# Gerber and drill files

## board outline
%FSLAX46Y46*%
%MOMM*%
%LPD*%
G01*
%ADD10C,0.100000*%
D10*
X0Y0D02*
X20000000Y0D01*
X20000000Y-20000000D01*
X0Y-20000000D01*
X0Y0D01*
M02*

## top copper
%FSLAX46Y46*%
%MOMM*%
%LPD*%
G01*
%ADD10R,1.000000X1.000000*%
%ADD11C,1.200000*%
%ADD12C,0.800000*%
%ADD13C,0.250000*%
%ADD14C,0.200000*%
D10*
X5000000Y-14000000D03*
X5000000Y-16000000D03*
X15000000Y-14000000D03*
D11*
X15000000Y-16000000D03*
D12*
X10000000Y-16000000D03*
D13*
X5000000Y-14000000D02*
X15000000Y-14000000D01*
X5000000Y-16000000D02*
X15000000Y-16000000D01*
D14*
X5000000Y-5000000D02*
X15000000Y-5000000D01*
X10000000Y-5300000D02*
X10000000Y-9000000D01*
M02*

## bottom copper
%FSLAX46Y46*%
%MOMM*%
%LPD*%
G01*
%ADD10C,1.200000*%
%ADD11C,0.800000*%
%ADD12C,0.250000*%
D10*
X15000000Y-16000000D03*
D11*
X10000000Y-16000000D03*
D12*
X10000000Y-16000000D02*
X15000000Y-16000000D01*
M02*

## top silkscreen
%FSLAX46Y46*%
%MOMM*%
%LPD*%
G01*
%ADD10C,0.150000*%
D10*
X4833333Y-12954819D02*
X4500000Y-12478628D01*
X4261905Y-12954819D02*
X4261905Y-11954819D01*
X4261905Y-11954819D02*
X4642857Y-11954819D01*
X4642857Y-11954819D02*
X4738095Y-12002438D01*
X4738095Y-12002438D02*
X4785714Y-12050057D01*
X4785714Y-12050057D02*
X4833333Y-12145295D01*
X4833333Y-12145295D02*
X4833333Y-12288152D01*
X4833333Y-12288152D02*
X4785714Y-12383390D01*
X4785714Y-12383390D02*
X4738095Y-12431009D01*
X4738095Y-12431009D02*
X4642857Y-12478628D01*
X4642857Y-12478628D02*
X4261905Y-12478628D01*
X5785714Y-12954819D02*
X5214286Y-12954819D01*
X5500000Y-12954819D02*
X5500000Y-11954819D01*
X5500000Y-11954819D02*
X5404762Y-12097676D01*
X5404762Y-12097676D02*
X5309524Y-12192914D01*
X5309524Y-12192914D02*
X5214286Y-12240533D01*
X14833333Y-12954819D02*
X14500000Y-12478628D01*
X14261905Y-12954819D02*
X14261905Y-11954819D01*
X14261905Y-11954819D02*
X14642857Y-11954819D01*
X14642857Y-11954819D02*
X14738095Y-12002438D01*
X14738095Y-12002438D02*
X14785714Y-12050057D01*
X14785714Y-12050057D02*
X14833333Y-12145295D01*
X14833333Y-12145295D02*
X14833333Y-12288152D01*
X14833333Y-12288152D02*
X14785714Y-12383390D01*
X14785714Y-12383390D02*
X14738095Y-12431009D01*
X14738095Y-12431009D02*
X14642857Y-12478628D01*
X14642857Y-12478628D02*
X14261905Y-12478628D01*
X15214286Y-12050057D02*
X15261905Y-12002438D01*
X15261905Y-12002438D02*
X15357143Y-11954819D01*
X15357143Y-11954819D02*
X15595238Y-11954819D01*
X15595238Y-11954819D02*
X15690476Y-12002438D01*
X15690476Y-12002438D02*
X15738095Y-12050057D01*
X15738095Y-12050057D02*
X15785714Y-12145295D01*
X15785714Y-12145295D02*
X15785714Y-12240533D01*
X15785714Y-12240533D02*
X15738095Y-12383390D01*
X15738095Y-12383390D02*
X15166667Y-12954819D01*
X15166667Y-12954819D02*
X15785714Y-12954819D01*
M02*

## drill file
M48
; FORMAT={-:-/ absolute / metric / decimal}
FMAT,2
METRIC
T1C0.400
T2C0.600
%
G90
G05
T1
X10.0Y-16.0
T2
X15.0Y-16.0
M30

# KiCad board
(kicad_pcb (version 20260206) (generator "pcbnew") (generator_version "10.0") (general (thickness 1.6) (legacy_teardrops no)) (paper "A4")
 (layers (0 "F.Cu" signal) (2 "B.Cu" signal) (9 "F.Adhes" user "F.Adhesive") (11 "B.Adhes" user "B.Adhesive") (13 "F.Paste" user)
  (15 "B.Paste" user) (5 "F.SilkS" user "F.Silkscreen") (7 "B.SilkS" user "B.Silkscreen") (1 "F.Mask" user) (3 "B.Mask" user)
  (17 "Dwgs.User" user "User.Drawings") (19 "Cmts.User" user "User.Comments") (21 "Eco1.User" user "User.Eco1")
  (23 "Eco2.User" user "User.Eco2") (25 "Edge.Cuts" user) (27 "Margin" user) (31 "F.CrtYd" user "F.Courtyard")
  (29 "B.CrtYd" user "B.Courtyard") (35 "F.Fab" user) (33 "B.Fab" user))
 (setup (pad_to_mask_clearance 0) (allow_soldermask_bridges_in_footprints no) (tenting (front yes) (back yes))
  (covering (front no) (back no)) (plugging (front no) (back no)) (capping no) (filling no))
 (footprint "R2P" (layer "F.Cu") (at 5 15)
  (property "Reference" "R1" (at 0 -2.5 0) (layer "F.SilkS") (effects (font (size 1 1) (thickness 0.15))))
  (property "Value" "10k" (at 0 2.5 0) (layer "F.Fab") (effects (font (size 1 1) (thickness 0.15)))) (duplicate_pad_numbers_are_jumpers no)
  (pad "1" smd rect (at 0 -1) (size 1 1) (layers "F.Cu" "F.Mask" "F.Paste") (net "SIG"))
  (pad "2" smd rect (at 0 1) (size 1 1) (layers "F.Cu" "F.Mask" "F.Paste") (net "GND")))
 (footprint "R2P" (layer "F.Cu") (at 15 15)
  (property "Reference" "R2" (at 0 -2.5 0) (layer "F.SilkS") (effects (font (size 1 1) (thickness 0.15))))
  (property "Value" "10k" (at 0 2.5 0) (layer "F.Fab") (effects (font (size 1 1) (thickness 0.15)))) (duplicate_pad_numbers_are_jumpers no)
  (pad "1" smd rect (at 0 -1) (size 1 1) (layers "F.Cu" "F.Mask" "F.Paste") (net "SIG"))
  (pad "2" thru_hole circle (at 0 1) (size 1.2 1.2) (drill 0.6) (layers "*.Cu" "*.Mask") (remove_unused_layers no) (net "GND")))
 (gr_rect (start 0 0) (end 20 20) (stroke (width 0.1) (type solid)) (fill no) (layer "Edge.Cuts"))
 (segment (start 5 14) (end 15 14) (width 0.25) (layer "F.Cu") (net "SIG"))
 (segment (start 5 16) (end 15 16) (width 0.25) (layer "F.Cu") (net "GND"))
 (via (at 10 16) (size 0.8) (drill 0.4) (layers "F.Cu" "B.Cu") (capping no) (covering (front no) (back no)) (plugging (front no) (back no))
  (filling no) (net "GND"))
 (segment (start 10 16) (end 15 16) (width 0.25) (layer "B.Cu") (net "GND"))
 (segment (start 5 5) (end 15 5) (width 0.2) (layer "F.Cu") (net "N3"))
 (segment (start 10 5.3) (end 10 9) (width 0.2) (layer "F.Cu") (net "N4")))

